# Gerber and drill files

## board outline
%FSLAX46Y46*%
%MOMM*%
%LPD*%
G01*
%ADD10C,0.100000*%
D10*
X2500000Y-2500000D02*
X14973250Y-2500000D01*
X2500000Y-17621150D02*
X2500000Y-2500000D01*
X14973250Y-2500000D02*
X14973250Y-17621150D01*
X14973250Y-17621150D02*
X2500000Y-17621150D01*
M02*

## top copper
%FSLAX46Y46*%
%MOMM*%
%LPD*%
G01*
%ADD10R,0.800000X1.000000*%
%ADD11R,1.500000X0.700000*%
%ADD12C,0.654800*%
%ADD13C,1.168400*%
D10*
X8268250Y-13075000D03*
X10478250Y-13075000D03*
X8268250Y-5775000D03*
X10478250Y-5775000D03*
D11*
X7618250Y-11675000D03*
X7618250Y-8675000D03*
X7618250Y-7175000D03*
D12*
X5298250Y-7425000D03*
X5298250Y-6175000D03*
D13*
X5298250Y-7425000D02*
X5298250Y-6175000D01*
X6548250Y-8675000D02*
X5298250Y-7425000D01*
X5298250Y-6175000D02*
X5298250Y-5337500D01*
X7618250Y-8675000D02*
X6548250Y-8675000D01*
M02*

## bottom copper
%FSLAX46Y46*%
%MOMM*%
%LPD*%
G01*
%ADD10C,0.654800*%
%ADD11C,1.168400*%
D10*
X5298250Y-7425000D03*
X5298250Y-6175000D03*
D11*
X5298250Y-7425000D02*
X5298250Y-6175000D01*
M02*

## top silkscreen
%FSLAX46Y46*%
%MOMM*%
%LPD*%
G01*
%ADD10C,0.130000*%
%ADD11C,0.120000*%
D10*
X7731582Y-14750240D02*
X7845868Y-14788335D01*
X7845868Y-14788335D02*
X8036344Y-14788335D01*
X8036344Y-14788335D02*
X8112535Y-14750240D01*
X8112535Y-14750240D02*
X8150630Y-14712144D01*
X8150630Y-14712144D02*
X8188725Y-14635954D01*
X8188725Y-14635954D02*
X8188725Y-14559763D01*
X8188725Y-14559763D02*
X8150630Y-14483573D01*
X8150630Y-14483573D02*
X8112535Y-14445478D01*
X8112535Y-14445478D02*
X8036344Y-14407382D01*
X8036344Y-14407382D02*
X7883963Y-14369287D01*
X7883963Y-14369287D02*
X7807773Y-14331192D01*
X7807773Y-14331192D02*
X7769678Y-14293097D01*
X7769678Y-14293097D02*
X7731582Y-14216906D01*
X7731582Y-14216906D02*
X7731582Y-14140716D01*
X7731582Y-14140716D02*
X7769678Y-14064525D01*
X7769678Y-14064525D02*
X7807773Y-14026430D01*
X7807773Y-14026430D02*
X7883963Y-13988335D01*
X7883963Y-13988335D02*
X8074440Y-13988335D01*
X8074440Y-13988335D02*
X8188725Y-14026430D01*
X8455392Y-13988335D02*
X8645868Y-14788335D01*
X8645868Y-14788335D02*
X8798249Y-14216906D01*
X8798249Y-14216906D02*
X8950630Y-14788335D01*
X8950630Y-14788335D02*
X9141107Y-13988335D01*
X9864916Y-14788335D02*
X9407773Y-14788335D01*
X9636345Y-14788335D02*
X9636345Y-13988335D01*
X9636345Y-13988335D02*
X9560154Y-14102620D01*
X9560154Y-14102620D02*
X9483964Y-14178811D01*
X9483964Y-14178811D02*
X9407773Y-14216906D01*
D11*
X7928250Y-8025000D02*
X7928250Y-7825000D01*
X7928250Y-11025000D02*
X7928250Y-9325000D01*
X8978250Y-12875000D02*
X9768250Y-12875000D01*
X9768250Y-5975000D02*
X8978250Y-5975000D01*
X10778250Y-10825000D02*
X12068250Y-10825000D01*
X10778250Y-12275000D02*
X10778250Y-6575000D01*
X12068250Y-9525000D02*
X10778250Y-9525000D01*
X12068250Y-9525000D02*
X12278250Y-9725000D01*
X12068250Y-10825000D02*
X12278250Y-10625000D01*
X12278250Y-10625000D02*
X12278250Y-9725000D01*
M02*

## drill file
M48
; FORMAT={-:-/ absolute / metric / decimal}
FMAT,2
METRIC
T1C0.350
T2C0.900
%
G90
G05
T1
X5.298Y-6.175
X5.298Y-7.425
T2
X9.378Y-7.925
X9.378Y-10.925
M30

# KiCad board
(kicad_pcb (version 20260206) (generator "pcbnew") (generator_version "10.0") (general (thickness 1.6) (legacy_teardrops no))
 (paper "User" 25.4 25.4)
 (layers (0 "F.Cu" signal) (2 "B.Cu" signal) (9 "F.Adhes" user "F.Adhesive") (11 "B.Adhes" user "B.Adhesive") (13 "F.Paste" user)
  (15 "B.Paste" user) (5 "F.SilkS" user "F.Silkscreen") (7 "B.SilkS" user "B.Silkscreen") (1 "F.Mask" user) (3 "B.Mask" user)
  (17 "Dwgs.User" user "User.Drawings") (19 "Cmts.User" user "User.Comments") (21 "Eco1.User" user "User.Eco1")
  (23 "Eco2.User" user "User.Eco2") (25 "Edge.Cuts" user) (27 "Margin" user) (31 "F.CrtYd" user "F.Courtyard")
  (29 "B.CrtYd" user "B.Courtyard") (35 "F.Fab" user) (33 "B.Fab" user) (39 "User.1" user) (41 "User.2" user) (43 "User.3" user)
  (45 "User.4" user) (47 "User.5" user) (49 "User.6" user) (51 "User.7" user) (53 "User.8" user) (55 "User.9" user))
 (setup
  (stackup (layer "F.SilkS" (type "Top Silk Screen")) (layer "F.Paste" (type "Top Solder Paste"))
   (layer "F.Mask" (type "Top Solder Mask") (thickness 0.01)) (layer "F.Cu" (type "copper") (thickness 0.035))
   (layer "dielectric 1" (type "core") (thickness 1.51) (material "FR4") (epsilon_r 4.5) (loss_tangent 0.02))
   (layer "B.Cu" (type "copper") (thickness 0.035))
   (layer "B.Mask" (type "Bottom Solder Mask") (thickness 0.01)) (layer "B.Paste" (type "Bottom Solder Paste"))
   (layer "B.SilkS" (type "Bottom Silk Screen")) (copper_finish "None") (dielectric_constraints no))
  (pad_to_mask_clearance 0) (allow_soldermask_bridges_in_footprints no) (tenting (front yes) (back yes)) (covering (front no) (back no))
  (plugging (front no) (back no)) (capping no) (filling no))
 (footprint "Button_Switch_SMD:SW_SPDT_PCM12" (layer "F.Cu") (at 9.04825 9.425 90)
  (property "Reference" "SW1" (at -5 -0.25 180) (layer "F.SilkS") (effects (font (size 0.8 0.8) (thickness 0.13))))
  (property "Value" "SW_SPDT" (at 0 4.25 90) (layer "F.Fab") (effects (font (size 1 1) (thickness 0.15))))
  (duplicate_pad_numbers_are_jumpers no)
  (fp_line (start 1.4 -1.12) (end 1.6 -1.12) (stroke (width 0.12) (type solid)) (layer "F.SilkS"))
  (fp_line (start -1.6 -1.12) (end 0.1 -1.12) (stroke (width 0.12) (type solid)) (layer "F.SilkS"))
  (fp_line (start -3.45 -0.07) (end -3.45 0.72) (stroke (width 0.12) (type solid)) (layer "F.SilkS"))
  (fp_line (start 3.45 0.72) (end 3.45 -0.07) (stroke (width 0.12) (type solid)) (layer "F.SilkS"))
  (fp_line (start -1.4 1.73) (end -1.4 3.02) (stroke (width 0.12) (type solid)) (layer "F.SilkS"))
  (fp_line (start -2.85 1.73) (end 2.85 1.73) (stroke (width 0.12) (type solid)) (layer "F.SilkS"))
  (fp_line (start -0.1 3.02) (end -0.1 1.73) (stroke (width 0.12) (type solid)) (layer "F.SilkS"))
  (fp_line (start -0.1 3.02) (end -0.3 3.23) (stroke (width 0.12) (type solid)) (layer "F.SilkS"))
  (fp_line (start -1.4 3.02) (end -1.2 3.23) (stroke (width 0.12) (type solid)) (layer "F.SilkS"))
  (fp_line (start -1.2 3.23) (end -0.3 3.23) (stroke (width 0.12) (type solid)) (layer "F.SilkS"))
  (pad "" smd rect (at -3.65 -0.78 90) (size 1 0.8) (layers "F.Cu" "F.Mask" "F.Paste"))
  (pad "" smd rect (at -3.65 1.43 90) (size 1 0.8) (layers "F.Cu" "F.Mask" "F.Paste"))
  (pad "" np_thru_hole circle (at -1.5 0.33 90) (size 0.9 0.9) (drill 0.9) (layers "*.Cu" "*.Mask"))
  (pad "" np_thru_hole circle (at 1.5 0.33 90) (size 0.9 0.9) (drill 0.9) (layers "*.Cu" "*.Mask"))
  (pad "" smd rect (at 3.65 -0.78 90) (size 1 0.8) (layers "F.Cu" "F.Mask" "F.Paste"))
  (pad "" smd rect (at 3.65 1.43 90) (size 1 0.8) (layers "F.Cu" "F.Mask" "F.Paste"))
  (pad "1" smd rect (at -2.25 -1.43 90) (size 0.7 1.5) (layers "F.Cu" "F.Mask" "F.Paste") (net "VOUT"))
  (pad "2" smd rect (at 0.75 -1.43 90) (size 0.7 1.5) (layers "F.Cu" "F.Mask" "F.Paste") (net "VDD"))
  (pad "3" smd rect (at 2.25 -1.43 90) (size 0.7 1.5) (layers "F.Cu" "F.Mask" "F.Paste") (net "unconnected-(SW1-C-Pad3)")))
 (gr_line (start 2.5 2.5) (end 14.97325 2.5) (stroke (width 0.1) (type default)) (layer "Edge.Cuts"))
 (gr_line (start 2.5 17.62115) (end 2.5 2.5) (stroke (width 0.1) (type default)) (layer "Edge.Cuts"))
 (gr_line (start 14.97325 2.5) (end 14.97325 17.62115) (stroke (width 0.1) (type default)) (layer "Edge.Cuts"))
 (gr_line (start 14.97325 17.62115) (end 2.5 17.62115) (stroke (width 0.1) (type default)) (layer "Edge.Cuts"))
 (segment (start 5.29825 7.425) (end 5.29825 6.175) (width 1.1684) (layer "F.Cu") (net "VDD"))
 (segment (start 6.54825 8.675) (end 5.29825 7.425) (width 1.1684) (layer "F.Cu") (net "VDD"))
 (segment (start 5.29825 6.175) (end 5.29825 5.3375) (width 1.1684) (layer "F.Cu") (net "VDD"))
 (segment (start 7.61825 8.675) (end 6.54825 8.675) (width 1.1684) (layer "F.Cu") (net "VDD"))
 (via (at 5.29825 7.425) (size 0.6548) (drill 0.35) (layers "F.Cu" "B.Cu") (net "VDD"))
 (via (at 5.29825 6.175) (size 0.6548) (drill 0.35) (layers "F.Cu" "B.Cu") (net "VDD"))
 (segment (start 5.29825 7.425) (end 5.29825 6.175) (width 1.1684) (layer "B.Cu") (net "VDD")))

